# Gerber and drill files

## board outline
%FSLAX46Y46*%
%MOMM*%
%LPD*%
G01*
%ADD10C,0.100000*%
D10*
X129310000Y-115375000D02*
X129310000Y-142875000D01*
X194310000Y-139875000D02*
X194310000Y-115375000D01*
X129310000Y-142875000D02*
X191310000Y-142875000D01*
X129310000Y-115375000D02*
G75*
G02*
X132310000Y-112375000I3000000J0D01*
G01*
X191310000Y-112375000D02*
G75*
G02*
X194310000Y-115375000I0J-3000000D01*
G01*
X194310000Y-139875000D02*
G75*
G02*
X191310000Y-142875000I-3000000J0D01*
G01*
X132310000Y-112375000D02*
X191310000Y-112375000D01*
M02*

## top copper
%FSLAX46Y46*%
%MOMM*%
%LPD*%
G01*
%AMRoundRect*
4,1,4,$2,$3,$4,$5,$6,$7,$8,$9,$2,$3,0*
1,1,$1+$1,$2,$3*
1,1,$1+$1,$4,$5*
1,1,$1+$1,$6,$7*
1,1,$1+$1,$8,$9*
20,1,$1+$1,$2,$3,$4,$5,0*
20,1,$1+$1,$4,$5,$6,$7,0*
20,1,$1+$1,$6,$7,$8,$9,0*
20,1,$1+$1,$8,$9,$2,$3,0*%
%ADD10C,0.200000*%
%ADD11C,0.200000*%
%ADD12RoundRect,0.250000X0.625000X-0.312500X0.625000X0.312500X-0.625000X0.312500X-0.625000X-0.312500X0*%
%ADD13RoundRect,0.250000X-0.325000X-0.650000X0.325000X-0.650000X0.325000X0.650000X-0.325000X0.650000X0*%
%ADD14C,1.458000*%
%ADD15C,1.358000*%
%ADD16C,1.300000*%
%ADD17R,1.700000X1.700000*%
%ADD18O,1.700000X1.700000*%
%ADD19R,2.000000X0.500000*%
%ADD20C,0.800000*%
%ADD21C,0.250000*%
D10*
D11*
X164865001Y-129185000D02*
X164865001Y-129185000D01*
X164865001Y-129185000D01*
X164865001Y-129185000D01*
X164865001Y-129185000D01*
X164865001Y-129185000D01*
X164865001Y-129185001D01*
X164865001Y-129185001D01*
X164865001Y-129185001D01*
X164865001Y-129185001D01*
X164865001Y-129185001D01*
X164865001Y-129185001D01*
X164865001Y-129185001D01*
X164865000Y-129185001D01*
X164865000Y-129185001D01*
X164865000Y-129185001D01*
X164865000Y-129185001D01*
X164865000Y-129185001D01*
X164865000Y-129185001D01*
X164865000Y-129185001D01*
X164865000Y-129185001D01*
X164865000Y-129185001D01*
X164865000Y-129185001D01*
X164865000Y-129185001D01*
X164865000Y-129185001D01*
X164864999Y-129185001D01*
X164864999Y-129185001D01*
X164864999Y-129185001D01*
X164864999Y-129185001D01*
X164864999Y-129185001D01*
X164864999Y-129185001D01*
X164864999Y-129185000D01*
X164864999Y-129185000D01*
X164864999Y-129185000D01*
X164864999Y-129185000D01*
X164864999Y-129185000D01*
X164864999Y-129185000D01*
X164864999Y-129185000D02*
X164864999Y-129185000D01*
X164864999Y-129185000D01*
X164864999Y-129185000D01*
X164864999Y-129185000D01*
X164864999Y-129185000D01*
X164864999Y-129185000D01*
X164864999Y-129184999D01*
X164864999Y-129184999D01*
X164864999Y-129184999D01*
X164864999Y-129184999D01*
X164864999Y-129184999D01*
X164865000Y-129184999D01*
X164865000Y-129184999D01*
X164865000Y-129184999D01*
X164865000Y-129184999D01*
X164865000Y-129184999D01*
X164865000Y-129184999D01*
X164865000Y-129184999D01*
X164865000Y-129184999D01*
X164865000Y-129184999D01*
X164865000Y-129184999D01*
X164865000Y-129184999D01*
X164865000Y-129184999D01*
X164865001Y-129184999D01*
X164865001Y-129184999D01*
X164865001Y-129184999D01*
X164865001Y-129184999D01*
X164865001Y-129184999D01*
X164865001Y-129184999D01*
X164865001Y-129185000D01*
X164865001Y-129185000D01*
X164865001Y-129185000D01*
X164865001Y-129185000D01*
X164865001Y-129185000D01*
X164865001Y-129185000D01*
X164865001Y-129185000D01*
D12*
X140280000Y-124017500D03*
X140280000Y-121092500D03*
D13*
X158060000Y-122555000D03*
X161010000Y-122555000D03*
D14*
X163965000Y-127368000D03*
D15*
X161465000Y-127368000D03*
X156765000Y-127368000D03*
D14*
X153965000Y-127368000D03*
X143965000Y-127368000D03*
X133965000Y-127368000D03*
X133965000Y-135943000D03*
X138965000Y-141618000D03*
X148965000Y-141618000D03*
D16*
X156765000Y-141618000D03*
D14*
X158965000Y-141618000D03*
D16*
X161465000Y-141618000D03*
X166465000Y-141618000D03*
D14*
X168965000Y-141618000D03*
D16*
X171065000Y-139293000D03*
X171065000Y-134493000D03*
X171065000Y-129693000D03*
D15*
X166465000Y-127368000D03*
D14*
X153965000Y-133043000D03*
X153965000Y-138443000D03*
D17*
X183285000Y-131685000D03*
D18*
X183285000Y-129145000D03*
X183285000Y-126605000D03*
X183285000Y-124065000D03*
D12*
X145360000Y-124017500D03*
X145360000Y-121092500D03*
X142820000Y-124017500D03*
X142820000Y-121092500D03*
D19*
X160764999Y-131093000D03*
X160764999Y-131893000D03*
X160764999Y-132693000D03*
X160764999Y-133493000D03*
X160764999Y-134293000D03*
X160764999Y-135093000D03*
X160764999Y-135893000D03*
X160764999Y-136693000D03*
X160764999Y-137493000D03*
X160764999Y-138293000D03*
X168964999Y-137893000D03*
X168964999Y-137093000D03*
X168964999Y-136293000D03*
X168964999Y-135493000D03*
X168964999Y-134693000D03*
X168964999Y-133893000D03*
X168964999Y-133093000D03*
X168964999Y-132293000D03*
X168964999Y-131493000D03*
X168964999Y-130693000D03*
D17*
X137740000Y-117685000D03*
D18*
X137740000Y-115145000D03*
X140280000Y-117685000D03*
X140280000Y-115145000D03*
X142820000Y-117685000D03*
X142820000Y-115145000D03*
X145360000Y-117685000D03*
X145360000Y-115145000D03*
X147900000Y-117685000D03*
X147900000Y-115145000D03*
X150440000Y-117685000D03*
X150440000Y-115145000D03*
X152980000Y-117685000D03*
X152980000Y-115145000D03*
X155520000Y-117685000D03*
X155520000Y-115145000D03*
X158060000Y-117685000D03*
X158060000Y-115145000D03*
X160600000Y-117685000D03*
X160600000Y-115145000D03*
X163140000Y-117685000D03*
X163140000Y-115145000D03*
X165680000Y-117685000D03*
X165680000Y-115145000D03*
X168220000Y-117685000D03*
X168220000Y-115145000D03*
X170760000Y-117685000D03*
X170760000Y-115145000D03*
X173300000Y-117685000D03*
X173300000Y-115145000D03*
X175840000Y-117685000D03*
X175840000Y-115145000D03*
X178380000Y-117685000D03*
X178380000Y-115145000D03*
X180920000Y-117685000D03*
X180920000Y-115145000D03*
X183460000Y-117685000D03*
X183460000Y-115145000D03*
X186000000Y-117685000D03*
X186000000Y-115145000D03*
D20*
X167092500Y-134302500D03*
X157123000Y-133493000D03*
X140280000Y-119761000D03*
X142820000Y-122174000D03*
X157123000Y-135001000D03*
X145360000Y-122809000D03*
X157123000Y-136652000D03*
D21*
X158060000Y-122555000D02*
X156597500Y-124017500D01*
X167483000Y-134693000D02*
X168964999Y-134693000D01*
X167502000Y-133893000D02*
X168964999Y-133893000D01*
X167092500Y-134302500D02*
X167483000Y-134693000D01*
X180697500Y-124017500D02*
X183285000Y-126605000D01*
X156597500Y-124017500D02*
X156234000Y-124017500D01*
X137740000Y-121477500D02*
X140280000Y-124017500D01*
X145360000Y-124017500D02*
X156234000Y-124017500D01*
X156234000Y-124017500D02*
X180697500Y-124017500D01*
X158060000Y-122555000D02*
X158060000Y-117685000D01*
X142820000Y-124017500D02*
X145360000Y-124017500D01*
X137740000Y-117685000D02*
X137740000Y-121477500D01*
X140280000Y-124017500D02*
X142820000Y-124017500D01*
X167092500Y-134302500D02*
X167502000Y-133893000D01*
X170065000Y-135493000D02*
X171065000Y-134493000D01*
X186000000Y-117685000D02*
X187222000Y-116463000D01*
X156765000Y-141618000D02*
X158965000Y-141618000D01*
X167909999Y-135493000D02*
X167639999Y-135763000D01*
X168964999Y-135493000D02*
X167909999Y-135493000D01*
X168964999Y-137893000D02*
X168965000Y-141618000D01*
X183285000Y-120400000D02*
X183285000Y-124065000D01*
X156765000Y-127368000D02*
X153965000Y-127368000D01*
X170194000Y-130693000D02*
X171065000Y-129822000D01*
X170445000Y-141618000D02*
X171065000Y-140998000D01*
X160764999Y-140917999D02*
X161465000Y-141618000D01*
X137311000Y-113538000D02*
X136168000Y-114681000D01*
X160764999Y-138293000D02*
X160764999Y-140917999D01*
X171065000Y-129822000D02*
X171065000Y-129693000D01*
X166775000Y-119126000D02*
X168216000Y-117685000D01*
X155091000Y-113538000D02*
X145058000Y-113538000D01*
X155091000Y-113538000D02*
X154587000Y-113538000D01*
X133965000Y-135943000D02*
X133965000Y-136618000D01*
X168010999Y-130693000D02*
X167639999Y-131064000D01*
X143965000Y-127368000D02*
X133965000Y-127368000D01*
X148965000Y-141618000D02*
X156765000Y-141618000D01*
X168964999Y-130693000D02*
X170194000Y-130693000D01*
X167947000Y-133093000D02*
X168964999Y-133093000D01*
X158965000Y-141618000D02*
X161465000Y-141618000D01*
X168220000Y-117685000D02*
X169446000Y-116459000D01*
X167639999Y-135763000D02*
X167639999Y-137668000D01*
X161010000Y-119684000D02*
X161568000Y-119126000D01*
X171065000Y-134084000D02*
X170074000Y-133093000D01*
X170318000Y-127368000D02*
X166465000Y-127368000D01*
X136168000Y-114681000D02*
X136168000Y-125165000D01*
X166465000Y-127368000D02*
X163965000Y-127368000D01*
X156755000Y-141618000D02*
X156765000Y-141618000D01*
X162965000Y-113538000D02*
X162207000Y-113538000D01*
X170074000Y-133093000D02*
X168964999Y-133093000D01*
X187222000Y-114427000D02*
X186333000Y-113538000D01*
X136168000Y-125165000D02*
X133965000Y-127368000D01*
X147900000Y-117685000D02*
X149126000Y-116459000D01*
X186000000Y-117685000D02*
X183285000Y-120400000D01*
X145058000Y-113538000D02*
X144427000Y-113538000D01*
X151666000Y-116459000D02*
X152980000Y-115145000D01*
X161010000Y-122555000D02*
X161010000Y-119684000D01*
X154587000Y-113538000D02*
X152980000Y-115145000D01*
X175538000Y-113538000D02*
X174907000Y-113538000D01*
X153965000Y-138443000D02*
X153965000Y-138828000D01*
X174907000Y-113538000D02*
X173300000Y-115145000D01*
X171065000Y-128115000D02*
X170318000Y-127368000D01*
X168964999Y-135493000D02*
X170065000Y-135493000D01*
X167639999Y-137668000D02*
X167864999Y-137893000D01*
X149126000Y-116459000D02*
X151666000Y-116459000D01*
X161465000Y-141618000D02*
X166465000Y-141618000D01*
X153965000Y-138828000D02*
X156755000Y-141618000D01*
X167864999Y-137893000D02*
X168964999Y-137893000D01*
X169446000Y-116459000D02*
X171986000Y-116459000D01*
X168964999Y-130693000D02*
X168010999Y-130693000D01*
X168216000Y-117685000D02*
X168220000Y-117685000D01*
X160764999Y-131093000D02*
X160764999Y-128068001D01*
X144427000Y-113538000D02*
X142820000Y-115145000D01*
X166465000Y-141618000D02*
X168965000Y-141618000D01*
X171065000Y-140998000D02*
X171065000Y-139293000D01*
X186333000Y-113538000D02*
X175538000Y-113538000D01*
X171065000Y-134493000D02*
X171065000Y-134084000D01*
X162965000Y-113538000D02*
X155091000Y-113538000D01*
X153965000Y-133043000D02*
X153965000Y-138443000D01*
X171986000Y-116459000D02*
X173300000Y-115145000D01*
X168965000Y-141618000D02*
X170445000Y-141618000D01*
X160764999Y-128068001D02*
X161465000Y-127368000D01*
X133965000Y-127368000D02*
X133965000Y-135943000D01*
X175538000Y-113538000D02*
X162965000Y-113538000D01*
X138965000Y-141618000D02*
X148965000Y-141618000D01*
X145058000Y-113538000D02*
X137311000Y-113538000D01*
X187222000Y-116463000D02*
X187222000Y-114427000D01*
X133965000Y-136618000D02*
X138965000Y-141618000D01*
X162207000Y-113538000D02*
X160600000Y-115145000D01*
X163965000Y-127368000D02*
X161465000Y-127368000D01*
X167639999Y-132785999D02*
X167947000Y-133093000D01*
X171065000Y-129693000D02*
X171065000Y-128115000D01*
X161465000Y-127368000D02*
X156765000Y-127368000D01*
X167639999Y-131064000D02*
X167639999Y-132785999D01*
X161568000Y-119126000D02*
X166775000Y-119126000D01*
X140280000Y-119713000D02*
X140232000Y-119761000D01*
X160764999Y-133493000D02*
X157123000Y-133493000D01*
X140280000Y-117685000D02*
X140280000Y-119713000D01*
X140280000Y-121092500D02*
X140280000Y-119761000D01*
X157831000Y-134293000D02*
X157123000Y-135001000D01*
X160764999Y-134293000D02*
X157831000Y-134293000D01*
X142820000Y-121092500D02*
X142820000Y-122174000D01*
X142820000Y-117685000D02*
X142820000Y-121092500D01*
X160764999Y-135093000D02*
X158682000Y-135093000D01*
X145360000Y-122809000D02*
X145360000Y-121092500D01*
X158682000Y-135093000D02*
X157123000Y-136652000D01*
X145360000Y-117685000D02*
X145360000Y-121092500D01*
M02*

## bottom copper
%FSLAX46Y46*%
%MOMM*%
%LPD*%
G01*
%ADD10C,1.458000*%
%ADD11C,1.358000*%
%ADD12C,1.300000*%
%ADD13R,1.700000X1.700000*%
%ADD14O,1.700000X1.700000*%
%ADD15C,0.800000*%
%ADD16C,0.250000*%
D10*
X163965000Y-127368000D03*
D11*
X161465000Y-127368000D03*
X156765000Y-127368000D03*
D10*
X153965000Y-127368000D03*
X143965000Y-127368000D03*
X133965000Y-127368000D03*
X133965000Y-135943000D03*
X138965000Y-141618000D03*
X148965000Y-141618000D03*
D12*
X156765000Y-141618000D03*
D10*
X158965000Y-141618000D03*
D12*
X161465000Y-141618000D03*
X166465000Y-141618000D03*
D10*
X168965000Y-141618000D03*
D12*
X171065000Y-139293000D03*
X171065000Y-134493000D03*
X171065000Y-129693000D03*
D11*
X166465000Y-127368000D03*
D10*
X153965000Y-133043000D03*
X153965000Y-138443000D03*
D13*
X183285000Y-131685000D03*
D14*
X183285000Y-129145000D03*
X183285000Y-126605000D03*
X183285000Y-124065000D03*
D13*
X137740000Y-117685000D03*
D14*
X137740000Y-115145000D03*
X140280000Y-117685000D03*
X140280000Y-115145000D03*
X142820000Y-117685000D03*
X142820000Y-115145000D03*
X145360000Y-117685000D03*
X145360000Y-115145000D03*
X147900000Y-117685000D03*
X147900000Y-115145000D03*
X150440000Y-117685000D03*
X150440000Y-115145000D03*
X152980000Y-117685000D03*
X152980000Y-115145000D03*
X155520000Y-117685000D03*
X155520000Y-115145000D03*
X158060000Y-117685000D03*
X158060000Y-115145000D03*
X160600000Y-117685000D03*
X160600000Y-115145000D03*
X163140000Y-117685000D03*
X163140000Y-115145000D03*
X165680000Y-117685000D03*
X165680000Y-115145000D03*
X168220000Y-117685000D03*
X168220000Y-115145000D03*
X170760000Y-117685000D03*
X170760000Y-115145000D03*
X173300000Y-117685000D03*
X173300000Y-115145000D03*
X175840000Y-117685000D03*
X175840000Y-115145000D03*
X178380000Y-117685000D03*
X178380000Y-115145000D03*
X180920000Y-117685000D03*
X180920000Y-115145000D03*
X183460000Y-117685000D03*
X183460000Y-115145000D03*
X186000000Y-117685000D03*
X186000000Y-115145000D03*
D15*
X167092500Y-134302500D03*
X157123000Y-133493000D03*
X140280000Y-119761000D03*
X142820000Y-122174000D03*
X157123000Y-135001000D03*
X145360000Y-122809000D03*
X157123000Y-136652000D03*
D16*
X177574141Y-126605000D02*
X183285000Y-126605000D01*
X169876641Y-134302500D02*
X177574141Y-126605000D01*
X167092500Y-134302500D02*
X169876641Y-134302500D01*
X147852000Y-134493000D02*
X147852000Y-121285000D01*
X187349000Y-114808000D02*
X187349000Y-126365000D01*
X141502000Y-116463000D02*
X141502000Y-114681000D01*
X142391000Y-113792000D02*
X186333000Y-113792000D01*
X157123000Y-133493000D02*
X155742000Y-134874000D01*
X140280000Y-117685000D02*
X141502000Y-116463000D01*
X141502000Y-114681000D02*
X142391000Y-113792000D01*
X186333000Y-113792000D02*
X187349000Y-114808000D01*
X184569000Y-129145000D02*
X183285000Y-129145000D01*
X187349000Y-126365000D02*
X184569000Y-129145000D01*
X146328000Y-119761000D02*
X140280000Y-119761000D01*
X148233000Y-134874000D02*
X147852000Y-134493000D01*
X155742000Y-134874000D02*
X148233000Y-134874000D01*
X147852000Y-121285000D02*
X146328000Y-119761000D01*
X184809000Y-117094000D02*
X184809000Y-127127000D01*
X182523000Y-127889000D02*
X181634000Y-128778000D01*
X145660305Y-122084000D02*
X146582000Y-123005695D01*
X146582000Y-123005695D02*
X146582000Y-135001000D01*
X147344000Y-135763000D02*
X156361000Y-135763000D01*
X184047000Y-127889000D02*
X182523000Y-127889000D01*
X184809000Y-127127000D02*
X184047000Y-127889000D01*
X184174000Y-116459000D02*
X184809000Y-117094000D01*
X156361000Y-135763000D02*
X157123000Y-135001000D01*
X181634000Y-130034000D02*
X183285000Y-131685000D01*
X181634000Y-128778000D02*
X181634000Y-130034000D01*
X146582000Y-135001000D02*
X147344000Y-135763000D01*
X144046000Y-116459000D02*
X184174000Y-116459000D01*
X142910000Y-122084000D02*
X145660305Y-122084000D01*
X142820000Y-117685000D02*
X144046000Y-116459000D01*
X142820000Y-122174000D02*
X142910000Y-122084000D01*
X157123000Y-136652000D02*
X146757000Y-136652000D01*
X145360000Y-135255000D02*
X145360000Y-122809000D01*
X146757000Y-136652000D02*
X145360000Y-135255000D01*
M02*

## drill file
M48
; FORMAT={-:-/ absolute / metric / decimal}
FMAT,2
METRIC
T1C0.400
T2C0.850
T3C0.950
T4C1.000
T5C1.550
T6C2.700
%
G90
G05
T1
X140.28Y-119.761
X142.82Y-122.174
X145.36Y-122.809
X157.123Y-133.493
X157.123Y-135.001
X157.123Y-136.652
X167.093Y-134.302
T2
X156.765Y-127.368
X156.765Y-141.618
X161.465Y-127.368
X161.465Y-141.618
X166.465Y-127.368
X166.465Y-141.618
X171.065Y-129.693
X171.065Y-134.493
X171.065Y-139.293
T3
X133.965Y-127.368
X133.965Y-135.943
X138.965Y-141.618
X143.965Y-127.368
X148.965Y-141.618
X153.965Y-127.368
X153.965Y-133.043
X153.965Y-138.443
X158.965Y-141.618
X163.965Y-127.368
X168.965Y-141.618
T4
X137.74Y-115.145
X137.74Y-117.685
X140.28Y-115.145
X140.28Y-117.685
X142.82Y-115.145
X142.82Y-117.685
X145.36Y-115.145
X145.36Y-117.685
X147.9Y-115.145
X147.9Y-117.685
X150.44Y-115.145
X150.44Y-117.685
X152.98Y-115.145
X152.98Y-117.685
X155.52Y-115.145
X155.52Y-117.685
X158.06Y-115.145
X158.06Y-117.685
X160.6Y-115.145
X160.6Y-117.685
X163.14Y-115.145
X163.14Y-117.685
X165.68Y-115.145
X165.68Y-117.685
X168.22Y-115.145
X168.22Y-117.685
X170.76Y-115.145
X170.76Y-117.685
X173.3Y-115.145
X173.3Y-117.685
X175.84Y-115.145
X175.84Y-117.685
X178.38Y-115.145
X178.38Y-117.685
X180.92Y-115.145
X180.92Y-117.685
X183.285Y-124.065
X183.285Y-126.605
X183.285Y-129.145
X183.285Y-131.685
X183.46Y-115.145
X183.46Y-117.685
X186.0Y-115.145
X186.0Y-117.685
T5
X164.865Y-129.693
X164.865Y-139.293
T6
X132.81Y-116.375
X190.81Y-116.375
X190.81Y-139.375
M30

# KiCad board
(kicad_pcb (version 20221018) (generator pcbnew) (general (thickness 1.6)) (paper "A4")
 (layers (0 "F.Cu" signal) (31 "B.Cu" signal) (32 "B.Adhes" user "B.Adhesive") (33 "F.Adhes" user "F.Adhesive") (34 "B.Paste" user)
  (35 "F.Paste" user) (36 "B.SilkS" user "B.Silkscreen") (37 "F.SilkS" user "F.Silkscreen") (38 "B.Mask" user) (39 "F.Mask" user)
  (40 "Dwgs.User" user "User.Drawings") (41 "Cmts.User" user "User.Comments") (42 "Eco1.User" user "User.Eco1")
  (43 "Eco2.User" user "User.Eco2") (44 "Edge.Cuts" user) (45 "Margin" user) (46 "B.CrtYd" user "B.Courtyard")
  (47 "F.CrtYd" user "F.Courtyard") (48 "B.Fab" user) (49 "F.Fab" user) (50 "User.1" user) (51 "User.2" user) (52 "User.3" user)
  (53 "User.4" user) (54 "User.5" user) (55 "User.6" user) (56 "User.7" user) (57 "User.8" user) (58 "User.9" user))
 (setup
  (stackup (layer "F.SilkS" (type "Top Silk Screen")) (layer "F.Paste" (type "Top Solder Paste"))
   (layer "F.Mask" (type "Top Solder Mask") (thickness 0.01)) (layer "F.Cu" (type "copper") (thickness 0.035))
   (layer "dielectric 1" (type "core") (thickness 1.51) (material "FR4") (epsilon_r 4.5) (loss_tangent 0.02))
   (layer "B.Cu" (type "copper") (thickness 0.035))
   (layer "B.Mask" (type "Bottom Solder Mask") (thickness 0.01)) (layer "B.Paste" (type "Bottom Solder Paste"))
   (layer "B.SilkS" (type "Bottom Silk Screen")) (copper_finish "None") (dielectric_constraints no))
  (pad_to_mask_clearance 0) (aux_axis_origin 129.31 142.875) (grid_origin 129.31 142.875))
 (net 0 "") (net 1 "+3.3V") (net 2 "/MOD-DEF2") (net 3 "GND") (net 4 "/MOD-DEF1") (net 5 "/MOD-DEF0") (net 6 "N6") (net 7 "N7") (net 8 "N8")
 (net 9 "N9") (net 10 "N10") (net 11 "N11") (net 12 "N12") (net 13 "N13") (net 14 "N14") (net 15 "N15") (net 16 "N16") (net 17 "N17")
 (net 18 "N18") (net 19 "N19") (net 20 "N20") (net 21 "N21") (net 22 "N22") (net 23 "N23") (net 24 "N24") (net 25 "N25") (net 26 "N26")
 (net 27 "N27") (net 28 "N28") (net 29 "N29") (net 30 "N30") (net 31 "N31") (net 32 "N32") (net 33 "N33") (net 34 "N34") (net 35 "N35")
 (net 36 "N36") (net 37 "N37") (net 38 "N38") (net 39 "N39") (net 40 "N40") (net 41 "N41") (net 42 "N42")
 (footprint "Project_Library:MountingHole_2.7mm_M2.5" (layer "F.Cu") (at 190.81 139.375)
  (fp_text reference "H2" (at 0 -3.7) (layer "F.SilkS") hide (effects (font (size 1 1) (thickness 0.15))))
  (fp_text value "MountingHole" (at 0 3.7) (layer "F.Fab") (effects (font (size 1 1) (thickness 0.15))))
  (pad "" np_thru_hole circle (at 0 0) (size 2.7 2.7) (drill 2.7) (layers "*.Cu" "*.Mask")))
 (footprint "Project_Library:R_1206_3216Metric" (layer "F.Cu") (at 140.28 122.555 90)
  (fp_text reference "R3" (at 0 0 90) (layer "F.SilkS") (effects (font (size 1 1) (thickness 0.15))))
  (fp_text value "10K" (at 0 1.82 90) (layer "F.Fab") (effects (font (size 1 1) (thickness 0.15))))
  (pad "1" smd roundrect (at -1.4625 0 90) (size 1.125 1.75) (layers "F.Cu" "F.Paste" "F.Mask") (roundrect_rratio 0.2222222222)
   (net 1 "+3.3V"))
  (pad "2" smd roundrect (at 1.4625 0 90) (size 1.125 1.75) (layers "F.Cu" "F.Paste" "F.Mask") (roundrect_rratio 0.2222222222)
   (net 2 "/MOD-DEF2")))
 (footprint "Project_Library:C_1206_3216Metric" (layer "F.Cu") (at 159.535 122.555)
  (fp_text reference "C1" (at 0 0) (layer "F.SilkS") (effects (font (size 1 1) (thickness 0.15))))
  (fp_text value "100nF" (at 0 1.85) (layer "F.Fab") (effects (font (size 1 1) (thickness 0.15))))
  (pad "1" smd roundrect (at -1.475 0) (size 1.15 1.8) (layers "F.Cu" "F.Paste" "F.Mask") (roundrect_rratio 0.2173913043) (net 1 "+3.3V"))
  (pad "2" smd roundrect (at 1.475 0) (size 1.15 1.8) (layers "F.Cu" "F.Paste" "F.Mask") (roundrect_rratio 0.2173913043) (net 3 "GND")))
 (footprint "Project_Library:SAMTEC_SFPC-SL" (layer "F.Cu") (at 164.865 129.698)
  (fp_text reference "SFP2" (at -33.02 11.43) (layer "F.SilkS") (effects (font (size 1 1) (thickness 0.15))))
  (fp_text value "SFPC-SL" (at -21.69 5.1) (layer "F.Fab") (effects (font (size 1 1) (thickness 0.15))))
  (pad "S1" thru_hole circle (at -0.9 -2.33 180) (size 1.458 1.458) (drill 0.95) (layers "*.Cu" "*.Mask") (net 3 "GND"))
  (pad "S2" thru_hole circle (at -3.4 -2.33 180) (size 1.358 1.358) (drill 0.85) (layers "*.Cu" "*.Mask") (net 3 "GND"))
  (pad "S3" thru_hole circle (at -8.1 -2.33 180) (size 1.358 1.358) (drill 0.85) (layers "*.Cu" "*.Mask") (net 3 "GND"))
  (pad "S4" thru_hole circle (at -10.9 -2.33 180) (size 1.458 1.458) (drill 0.95) (layers "*.Cu" "*.Mask") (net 3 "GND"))
  (pad "S5" thru_hole circle (at -20.9 -2.33 180) (size 1.458 1.458) (drill 0.95) (layers "*.Cu" "*.Mask") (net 3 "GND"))
  (pad "S6" thru_hole circle (at -30.9 -2.33 180) (size 1.458 1.458) (drill 0.95) (layers "*.Cu" "*.Mask") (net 3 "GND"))
  (pad "S7" thru_hole circle (at -30.9 6.245 180) (size 1.458 1.458) (drill 0.95) (layers "*.Cu" "*.Mask") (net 3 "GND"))
  (pad "S8" thru_hole circle (at -25.9 11.92 180) (size 1.458 1.458) (drill 0.95) (layers "*.Cu" "*.Mask") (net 3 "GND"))
  (pad "S9" thru_hole circle (at -15.9 11.92 180) (size 1.458 1.458) (drill 0.95) (layers "*.Cu" "*.Mask") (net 3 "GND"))
  (pad "S10" thru_hole circle (at -8.1 11.92 180) (size 1.3 1.3) (drill 0.85) (layers "*.Cu" "*.Mask") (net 3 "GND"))
  (pad "S11" thru_hole circle (at -5.9 11.92 180) (size 1.458 1.458) (drill 0.95) (layers "*.Cu" "*.Mask") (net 3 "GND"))
  (pad "S12" thru_hole circle (at -3.4 11.92 180) (size 1.3 1.3) (drill 0.85) (layers "*.Cu" "*.Mask") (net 3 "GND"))
  (pad "S13" thru_hole circle (at 1.6 11.92 180) (size 1.3 1.3) (drill 0.85) (layers "*.Cu" "*.Mask") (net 3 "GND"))
  (pad "S14" thru_hole circle (at 4.1 11.92 180) (size 1.458 1.458) (drill 0.95) (layers "*.Cu" "*.Mask") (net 3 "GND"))
  (pad "S15" thru_hole circle (at 6.2 9.595 180) (size 1.3 1.3) (drill 0.85) (layers "*.Cu" "*.Mask") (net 3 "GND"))
  (pad "S16" thru_hole circle (at 6.2 4.795 180) (size 1.3 1.3) (drill 0.85) (layers "*.Cu" "*.Mask") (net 3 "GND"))
  (pad "S17" thru_hole circle (at 6.2 -0.005 180) (size 1.3 1.3) (drill 0.85) (layers "*.Cu" "*.Mask") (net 3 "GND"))
  (pad "S18" thru_hole circle (at 1.6 -2.33 180) (size 1.358 1.358) (drill 0.85) (layers "*.Cu" "*.Mask") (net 3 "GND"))
  (pad "S19" thru_hole circle (at -10.9 3.345 180) (size 1.458 1.458) (drill 0.95) (layers "*.Cu" "*.Mask") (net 3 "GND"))
  (pad "S20" thru_hole circle (at -10.9 8.745 180) (size 1.458 1.458) (drill 0.95) (layers "*.Cu" "*.Mask") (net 3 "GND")))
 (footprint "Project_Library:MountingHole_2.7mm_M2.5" (layer "F.Cu") (at 132.81 116.375)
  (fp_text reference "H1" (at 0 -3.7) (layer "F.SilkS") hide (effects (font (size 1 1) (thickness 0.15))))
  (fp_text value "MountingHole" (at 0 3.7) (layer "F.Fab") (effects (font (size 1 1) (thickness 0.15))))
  (pad "" np_thru_hole circle (at 0 0) (size 2.7 2.7) (drill 2.7) (layers "*.Cu" "*.Mask")))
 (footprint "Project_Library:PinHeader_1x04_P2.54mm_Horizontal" (layer "F.Cu") (at 183.285 124.065)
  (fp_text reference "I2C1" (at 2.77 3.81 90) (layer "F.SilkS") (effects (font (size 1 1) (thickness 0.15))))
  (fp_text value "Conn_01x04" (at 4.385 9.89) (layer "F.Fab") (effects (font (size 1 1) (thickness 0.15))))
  (pad "1" thru_hole rect (at 0 7.62) (size 1.7 1.7) (drill 1) (layers "*.Cu" "*.Mask") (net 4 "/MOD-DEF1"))
  (pad "2" thru_hole oval (at 0 5.08) (size 1.7 1.7) (drill 1) (layers "*.Cu" "*.Mask") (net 2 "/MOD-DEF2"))
  (pad "3" thru_hole oval (at 0 2.54) (size 1.7 1.7) (drill 1) (layers "*.Cu" "*.Mask") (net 1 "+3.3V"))
  (pad "4" thru_hole oval (at 0 0) (size 1.7 1.7) (drill 1) (layers "*.Cu" "*.Mask") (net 3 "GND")))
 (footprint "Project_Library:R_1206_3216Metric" (layer "F.Cu") (at 145.36 122.555 90)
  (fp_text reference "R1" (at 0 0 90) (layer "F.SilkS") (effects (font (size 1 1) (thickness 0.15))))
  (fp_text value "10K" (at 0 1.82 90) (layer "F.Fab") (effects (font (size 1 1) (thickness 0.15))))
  (pad "1" smd roundrect (at -1.4625 0 90) (size 1.125 1.75) (layers "F.Cu" "F.Paste" "F.Mask") (roundrect_rratio 0.2222222222)
   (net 1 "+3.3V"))
  (pad "2" smd roundrect (at 1.4625 0 90) (size 1.125 1.75) (layers "F.Cu" "F.Paste" "F.Mask") (roundrect_rratio 0.2222222222)
   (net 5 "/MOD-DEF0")))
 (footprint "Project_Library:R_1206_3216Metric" (layer "F.Cu") (at 142.82 122.555 90)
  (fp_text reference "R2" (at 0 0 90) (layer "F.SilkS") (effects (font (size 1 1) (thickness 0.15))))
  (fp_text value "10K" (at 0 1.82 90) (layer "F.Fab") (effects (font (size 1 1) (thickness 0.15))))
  (pad "1" smd roundrect (at -1.4625 0 90) (size 1.125 1.75) (layers "F.Cu" "F.Paste" "F.Mask") (roundrect_rratio 0.2222222222)
   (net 1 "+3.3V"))
  (pad "2" smd roundrect (at 1.4625 0 90) (size 1.125 1.75) (layers "F.Cu" "F.Paste" "F.Mask") (roundrect_rratio 0.2222222222)
   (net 4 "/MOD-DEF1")))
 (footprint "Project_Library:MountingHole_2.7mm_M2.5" (layer "F.Cu") (at 190.81 116.375)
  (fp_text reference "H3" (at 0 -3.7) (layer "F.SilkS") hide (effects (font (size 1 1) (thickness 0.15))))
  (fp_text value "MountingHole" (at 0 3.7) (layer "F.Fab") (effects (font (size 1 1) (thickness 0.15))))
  (pad "" np_thru_hole circle (at 0 0) (size 2.7 2.7) (drill 2.7) (layers "*.Cu" "*.Mask")))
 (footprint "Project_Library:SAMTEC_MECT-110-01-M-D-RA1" (layer "F.Cu") (at 164.864999 129.693)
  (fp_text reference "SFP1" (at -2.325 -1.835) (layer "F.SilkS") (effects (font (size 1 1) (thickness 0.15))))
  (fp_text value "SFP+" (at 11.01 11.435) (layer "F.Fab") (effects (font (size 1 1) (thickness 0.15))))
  (pad "" np_thru_hole circle (at 0 0 270) (size 1.55 1.55) (drill 1.55) (layers "*.Cu" "*.Mask"))
  (pad "" np_thru_hole circle (at 0 9.6 270) (size 1.55 1.55) (drill 1.55) (layers "*.Cu" "*.Mask"))
  (pad "01" smd rect (at -4.1 1.4 270) (size 0.5 2) (layers "F.Cu" "F.Paste" "F.Mask") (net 3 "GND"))
  (pad "02" smd rect (at -4.1 2.2 270) (size 0.5 2) (layers "F.Cu" "F.Paste" "F.Mask") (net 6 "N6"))
  (pad "03" smd rect (at -4.1 3 270) (size 0.5 2) (layers "F.Cu" "F.Paste" "F.Mask") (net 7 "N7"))
  (pad "04" smd rect (at -4.1 3.8 270) (size 0.5 2) (layers "F.Cu" "F.Paste" "F.Mask") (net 2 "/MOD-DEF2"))
  (pad "05" smd rect (at -4.1 4.6 270) (size 0.5 2) (layers "F.Cu" "F.Paste" "F.Mask") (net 4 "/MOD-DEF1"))
  (pad "06" smd rect (at -4.1 5.4 270) (size 0.5 2) (layers "F.Cu" "F.Paste" "F.Mask") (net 5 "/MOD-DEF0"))
  (pad "07" smd rect (at -4.1 6.2 270) (size 0.5 2) (layers "F.Cu" "F.Paste" "F.Mask") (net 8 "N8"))
  (pad "08" smd rect (at -4.1 7 270) (size 0.5 2) (layers "F.Cu" "F.Paste" "F.Mask") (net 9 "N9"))
  (pad "09" smd rect (at -4.1 7.8 270) (size 0.5 2) (layers "F.Cu" "F.Paste" "F.Mask") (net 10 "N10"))
  (pad "10" smd rect (at -4.1 8.6 270) (size 0.5 2) (layers "F.Cu" "F.Paste" "F.Mask") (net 3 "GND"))
  (pad "11" smd rect (at 4.1 8.2 270) (size 0.5 2) (layers "F.Cu" "F.Paste" "F.Mask") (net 3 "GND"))
  (pad "12" smd rect (at 4.1 7.4 270) (size 0.5 2) (layers "F.Cu" "F.Paste" "F.Mask") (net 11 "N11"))
  (pad "13" smd rect (at 4.1 6.6 270) (size 0.5 2) (layers "F.Cu" "F.Paste" "F.Mask") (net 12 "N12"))
  (pad "14" smd rect (at 4.1 5.8 270) (size 0.5 2) (layers "F.Cu" "F.Paste" "F.Mask") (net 3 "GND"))
  (pad "15" smd rect (at 4.1 5 270) (size 0.5 2) (layers "F.Cu" "F.Paste" "F.Mask") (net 1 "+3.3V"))
  (pad "16" smd rect (at 4.1 4.2 270) (size 0.5 2) (layers "F.Cu" "F.Paste" "F.Mask") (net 1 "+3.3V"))
  (pad "17" smd rect (at 4.1 3.4 270) (size 0.5 2) (layers "F.Cu" "F.Paste" "F.Mask") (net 3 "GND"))
  (pad "18" smd rect (at 4.1 2.6 270) (size 0.5 2) (layers "F.Cu" "F.Paste" "F.Mask") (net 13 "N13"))
  (pad "19" smd rect (at 4.1 1.8 270) (size 0.5 2) (layers "F.Cu" "F.Paste" "F.Mask") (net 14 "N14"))
  (pad "20" smd rect (at 4.1 1 270) (size 0.5 2) (layers "F.Cu" "F.Paste" "F.Mask") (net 3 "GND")))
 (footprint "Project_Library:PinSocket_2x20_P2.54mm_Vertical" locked (layer "B.Cu") (at 161.81 116.375 180)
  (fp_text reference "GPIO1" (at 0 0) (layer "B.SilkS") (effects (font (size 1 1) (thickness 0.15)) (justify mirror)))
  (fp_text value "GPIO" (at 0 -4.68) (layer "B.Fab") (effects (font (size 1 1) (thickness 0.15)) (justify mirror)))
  (pad "1" thru_hole rect locked (at 24.07 -1.31 270) (size 1.7 1.7) (drill 1) (layers "*.Cu" "*.Mask") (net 1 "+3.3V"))
  (pad "2" thru_hole oval locked (at 24.07 1.23 270) (size 1.7 1.7) (drill 1) (layers "*.Cu" "*.Mask") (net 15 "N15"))
  (pad "3" thru_hole oval locked (at 21.53 -1.31 270) (size 1.7 1.7) (drill 1) (layers "*.Cu" "*.Mask") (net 2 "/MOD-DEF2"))
  (pad "4" thru_hole oval locked (at 21.53 1.23 270) (size 1.7 1.7) (drill 1) (layers "*.Cu" "*.Mask") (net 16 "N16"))
  (pad "5" thru_hole oval locked (at 18.99 -1.31 270) (size 1.7 1.7) (drill 1) (layers "*.Cu" "*.Mask") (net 4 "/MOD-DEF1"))
  (pad "6" thru_hole oval locked (at 18.99 1.23 270) (size 1.7 1.7) (drill 1) (layers "*.Cu" "*.Mask") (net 3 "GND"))
  (pad "7" thru_hole oval locked (at 16.45 -1.31 270) (size 1.7 1.7) (drill 1) (layers "*.Cu" "*.Mask") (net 5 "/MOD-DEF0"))
  (pad "8" thru_hole oval locked (at 16.45 1.23 270) (size 1.7 1.7) (drill 1) (layers "*.Cu" "*.Mask") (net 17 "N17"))
  (pad "9" thru_hole oval locked (at 13.91 -1.31 270) (size 1.7 1.7) (drill 1) (layers "*.Cu" "*.Mask") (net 3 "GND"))
  (pad "10" thru_hole oval locked (at 13.91 1.23 270) (size 1.7 1.7) (drill 1) (layers "*.Cu" "*.Mask") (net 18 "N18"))
  (pad "11" thru_hole oval locked (at 11.37 -1.31 270) (size 1.7 1.7) (drill 1) (layers "*.Cu" "*.Mask") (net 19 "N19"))
  (pad "12" thru_hole oval locked (at 11.37 1.23 270) (size 1.7 1.7) (drill 1) (layers "*.Cu" "*.Mask") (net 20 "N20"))
  (pad "13" thru_hole oval locked (at 8.83 -1.31 270) (size 1.7 1.7) (drill 1) (layers "*.Cu" "*.Mask") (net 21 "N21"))
  (pad "14" thru_hole oval locked (at 8.83 1.23 270) (size 1.7 1.7) (drill 1) (layers "*.Cu" "*.Mask") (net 3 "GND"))
  (pad "15" thru_hole oval locked (at 6.29 -1.31 270) (size 1.7 1.7) (drill 1) (layers "*.Cu" "*.Mask") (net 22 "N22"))
  (pad "16" thru_hole oval locked (at 6.29 1.23 270) (size 1.7 1.7) (drill 1) (layers "*.Cu" "*.Mask") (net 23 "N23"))
  (pad "17" thru_hole oval locked (at 3.75 -1.31 270) (size 1.7 1.7) (drill 1) (layers "*.Cu" "*.Mask") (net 1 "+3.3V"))
  (pad "18" thru_hole oval locked (at 3.75 1.23 270) (size 1.7 1.7) (drill 1) (layers "*.Cu" "*.Mask") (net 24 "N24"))
  (pad "19" thru_hole oval locked (at 1.21 -1.31 270) (size 1.7 1.7) (drill 1) (layers "*.Cu" "*.Mask") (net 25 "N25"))
  (pad "20" thru_hole oval locked (at 1.21 1.23 270) (size 1.7 1.7) (drill 1) (layers "*.Cu" "*.Mask") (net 3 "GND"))
  (pad "21" thru_hole oval locked (at -1.33 -1.31 270) (size 1.7 1.7) (drill 1) (layers "*.Cu" "*.Mask") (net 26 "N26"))
  (pad "22" thru_hole oval locked (at -1.33 1.23 270) (size 1.7 1.7) (drill 1) (layers "*.Cu" "*.Mask") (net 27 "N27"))
  (pad "23" thru_hole oval locked (at -3.87 -1.31 270) (size 1.7 1.7) (drill 1) (layers "*.Cu" "*.Mask") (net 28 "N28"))
  (pad "24" thru_hole oval locked (at -3.87 1.23 270) (size 1.7 1.7) (drill 1) (layers "*.Cu" "*.Mask") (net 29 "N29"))
  (pad "25" thru_hole oval locked (at -6.41 -1.31 270) (size 1.7 1.7) (drill 1) (layers "*.Cu" "*.Mask") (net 3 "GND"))
  (pad "26" thru_hole oval locked (at -6.41 1.23 270) (size 1.7 1.7) (drill 1) (layers "*.Cu" "*.Mask") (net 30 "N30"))
  (pad "27" thru_hole oval locked (at -8.95 -1.31 270) (size 1.7 1.7) (drill 1) (layers "*.Cu" "*.Mask") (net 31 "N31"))
  (pad "28" thru_hole oval locked (at -8.95 1.23 270) (size 1.7 1.7) (drill 1) (layers "*.Cu" "*.Mask") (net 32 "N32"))
  (pad "29" thru_hole oval locked (at -11.49 -1.31 270) (size 1.7 1.7) (drill 1) (layers "*.Cu" "*.Mask") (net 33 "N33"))
  (pad "30" thru_hole oval locked (at -11.49 1.23 270) (size 1.7 1.7) (drill 1) (layers "*.Cu" "*.Mask") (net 3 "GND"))
  (pad "31" thru_hole oval locked (at -14.03 -1.31 270) (size 1.7 1.7) (drill 1) (layers "*.Cu" "*.Mask") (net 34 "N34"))
  (pad "32" thru_hole oval locked (at -14.03 1.23 270) (size 1.7 1.7) (drill 1) (layers "*.Cu" "*.Mask") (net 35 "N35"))
  (pad "33" thru_hole oval locked (at -16.57 -1.31 270) (size 1.7 1.7) (drill 1) (layers "*.Cu" "*.Mask") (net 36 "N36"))
  (pad "34" thru_hole oval locked (at -16.57 1.23 270) (size 1.7 1.7) (drill 1) (layers "*.Cu" "*.Mask") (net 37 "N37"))
  (pad "35" thru_hole oval locked (at -19.11 -1.31 270) (size 1.7 1.7) (drill 1) (layers "*.Cu" "*.Mask") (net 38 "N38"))
  (pad "36" thru_hole oval locked (at -19.11 1.23 270) (size 1.7 1.7) (drill 1) (layers "*.Cu" "*.Mask") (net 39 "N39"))
  (pad "37" thru_hole oval locked (at -21.65 -1.31 270) (size 1.7 1.7) (drill 1) (layers "*.Cu" "*.Mask") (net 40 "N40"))
  (pad "38" thru_hole oval locked (at -21.65 1.23 270) (size 1.7 1.7) (drill 1) (layers "*.Cu" "*.Mask") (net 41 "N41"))
  (pad "39" thru_hole oval locked (at -24.19 -1.31 270) (size 1.7 1.7) (drill 1) (layers "*.Cu" "*.Mask") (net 3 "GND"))
  (pad "40" thru_hole oval locked (at -24.19 1.23 270) (size 1.7 1.7) (drill 1) (layers "*.Cu" "*.Mask") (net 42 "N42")))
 (gr_circle locked (center 164.865 129.185) (end 164.865001 129.185) (stroke (width 0.2) (type default)) (fill none) (layer "F.Cu"))
 (gr_line (start 129.31 115.375) (end 129.31 142.875) (stroke (width 0.1) (type solid)) (layer "Edge.Cuts"))
 (gr_line (start 194.31 139.875) (end 194.31 115.375) (stroke (width 0.1) (type solid)) (layer "Edge.Cuts"))
 (gr_line (start 129.31 142.875) (end 191.31 142.875) (stroke (width 0.1) (type solid)) (layer "Edge.Cuts"))
 (gr_arc (start 129.31 115.375) (mid 130.18868 113.25368) (end 132.31 112.375) (stroke (width 0.1) (type solid)) (layer "Edge.Cuts"))
 (gr_arc (start 191.31 112.375) (mid 193.43132 113.25368) (end 194.31 115.375) (stroke (width 0.1) (type solid)) (layer "Edge.Cuts"))
 (gr_arc (start 194.31 139.875) (mid 193.43132 141.99632) (end 191.31 142.875) (stroke (width 0.1) (type solid)) (layer "Edge.Cuts"))
 (gr_line (start 132.31 112.375) (end 191.31 112.375) (stroke (width 0.1) (type solid)) (layer "Edge.Cuts"))
 (segment (start 158.06 122.555) (end 156.5975 124.0175) (width 0.25) (layer "F.Cu") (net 1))
 (segment (start 167.483 134.693) (end 168.964999 134.693) (width 0.25) (layer "F.Cu") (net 1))
 (segment (start 167.502 133.893) (end 168.964999 133.893) (width 0.25) (layer "F.Cu") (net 1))
 (segment (start 167.0925 134.3025) (end 167.483 134.693) (width 0.25) (layer "F.Cu") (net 1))
 (segment (start 180.6975 124.0175) (end 183.285 126.605) (width 0.25) (layer "F.Cu") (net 1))
 (segment (start 156.5975 124.0175) (end 156.234 124.0175) (width 0.25) (layer "F.Cu") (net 1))
 (segment (start 137.74 121.4775) (end 140.28 124.0175) (width 0.25) (layer "F.Cu") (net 1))
 (segment (start 145.36 124.0175) (end 156.234 124.0175) (width 0.25) (layer "F.Cu") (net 1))
 (segment (start 156.234 124.0175) (end 180.6975 124.0175) (width 0.25) (layer "F.Cu") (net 1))
 (segment (start 158.06 122.555) (end 158.06 117.685) (width 0.25) (layer "F.Cu") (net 1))
 (segment (start 142.82 124.0175) (end 145.36 124.0175) (width 0.25) (layer "F.Cu") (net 1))
 (segment (start 137.74 117.685) (end 137.74 121.4775) (width 0.25) (layer "F.Cu") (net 1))
 (segment (start 140.28 124.0175) (end 142.82 124.0175) (width 0.25) (layer "F.Cu") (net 1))
 (segment (start 167.0925 134.3025) (end 167.502 133.893) (width 0.25) (layer "F.Cu") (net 1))
 (via (at 167.0925 134.3025) (size 0.8) (drill 0.4) (layers "F.Cu" "B.Cu") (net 1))
 (segment (start 177.574141 126.605) (end 183.285 126.605) (width 0.25) (layer "B.Cu") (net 1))
 (segment (start 169.876641 134.3025) (end 177.574141 126.605) (width 0.25) (layer "B.Cu") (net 1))
 (segment (start 167.0925 134.3025) (end 169.876641 134.3025) (width 0.25) (layer "B.Cu") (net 1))
 (segment (start 170.065 135.493) (end 171.065 134.493) (width 0.25) (layer "F.Cu") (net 3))
 (segment (start 186 117.685) (end 187.222 116.463) (width 0.25) (layer "F.Cu") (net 3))
 (segment (start 156.765 141.618) (end 158.965 141.618) (width 0.25) (layer "F.Cu") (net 3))
 (segment (start 167.909999 135.493) (end 167.639999 135.763) (width 0.25) (layer "F.Cu") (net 3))
 (segment (start 168.964999 135.493) (end 167.909999 135.493) (width 0.25) (layer "F.Cu") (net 3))
 (segment (start 168.964999 137.893) (end 168.965 141.618) (width 0.25) (layer "F.Cu") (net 3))
 (segment (start 183.285 120.4) (end 183.285 124.065) (width 0.25) (layer "F.Cu") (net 3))
 (segment (start 156.765 127.368) (end 153.965 127.368) (width 0.25) (layer "F.Cu") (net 3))
 (segment (start 170.194 130.693) (end 171.065 129.822) (width 0.25) (layer "F.Cu") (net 3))
 (segment (start 170.445 141.618) (end 171.065 140.998) (width 0.25) (layer "F.Cu") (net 3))
 (segment (start 160.764999 140.917999) (end 161.465 141.618) (width 0.25) (layer "F.Cu") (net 3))
 (segment (start 137.311 113.538) (end 136.168 114.681) (width 0.25) (layer "F.Cu") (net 3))
 (segment (start 160.764999 138.293) (end 160.764999 140.917999) (width 0.25) (layer "F.Cu") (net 3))
 (segment (start 171.065 129.822) (end 171.065 129.693) (width 0.25) (layer "F.Cu") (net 3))
 (segment (start 166.775 119.126) (end 168.216 117.685) (width 0.25) (layer "F.Cu") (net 3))
 (segment (start 155.091 113.538) (end 145.058 113.538) (width 0.25) (layer "F.Cu") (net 3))
 (segment (start 155.091 113.538) (end 154.587 113.538) (width 0.25) (layer "F.Cu") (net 3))
 (segment (start 133.965 135.943) (end 133.965 136.618) (width 0.25) (layer "F.Cu") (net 3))
 (segment (start 168.010999 130.693) (end 167.639999 131.064) (width 0.25) (layer "F.Cu") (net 3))
 (segment (start 143.965 127.368) (end 133.965 127.368) (width 0.25) (layer "F.Cu") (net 3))
 (segment (start 148.965 141.618) (end 156.765 141.618) (width 0.25) (layer "F.Cu") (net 3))
 (segment (start 168.964999 130.693) (end 170.194 130.693) (width 0.25) (layer "F.Cu") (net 3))
 (segment (start 167.947 133.093) (end 168.964999 133.093) (width 0.25) (layer "F.Cu") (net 3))
 (segment (start 158.965 141.618) (end 161.465 141.618) (width 0.25) (layer "F.Cu") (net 3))
 (segment (start 168.22 117.685) (end 169.446 116.459) (width 0.25) (layer "F.Cu") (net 3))
 (segment (start 167.639999 135.763) (end 167.639999 137.668) (width 0.25) (layer "F.Cu") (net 3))
 (segment (start 161.01 119.684) (end 161.568 119.126) (width 0.25) (layer "F.Cu") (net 3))
 (segment (start 171.065 134.084) (end 170.074 133.093) (width 0.25) (layer "F.Cu") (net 3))
 (segment (start 170.318 127.368) (end 166.465 127.368) (width 0.25) (layer "F.Cu") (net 3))
 (segment (start 136.168 114.681) (end 136.168 125.165) (width 0.25) (layer "F.Cu") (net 3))
 (segment (start 166.465 127.368) (end 163.965 127.368) (width 0.25) (layer "F.Cu") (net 3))
 (segment (start 156.755 141.618) (end 156.765 141.618) (width 0.25) (layer "F.Cu") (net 3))
 (segment (start 162.965 113.538) (end 162.207 113.538) (width 0.25) (layer "F.Cu") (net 3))
 (segment (start 170.074 133.093) (end 168.964999 133.093) (width 0.25) (layer "F.Cu") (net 3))
 (segment (start 187.222 114.427) (end 186.333 113.538) (width 0.25) (layer "F.Cu") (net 3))
 (segment (start 136.168 125.165) (end 133.965 127.368) (width 0.25) (layer "F.Cu") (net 3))
 (segment (start 147.9 117.685) (end 149.126 116.459) (width 0.25) (layer "F.Cu") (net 3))
 (segment (start 186 117.685) (end 183.285 120.4) (width 0.25) (layer "F.Cu") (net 3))
 (segment (start 145.058 113.538) (end 144.427 113.538) (width 0.25) (layer "F.Cu") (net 3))
 (segment (start 151.666 116.459) (end 152.98 115.145) (width 0.25) (layer "F.Cu") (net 3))
 (segment (start 161.01 122.555) (end 161.01 119.684) (width 0.25) (layer "F.Cu") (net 3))
 (segment (start 154.587 113.538) (end 152.98 115.145) (width 0.25) (layer "F.Cu") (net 3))
 (segment (start 175.538 113.538) (end 174.907 113.538) (width 0.25) (layer "F.Cu") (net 3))
 (segment (start 153.965 138.443) (end 153.965 138.828) (width 0.25) (layer "F.Cu") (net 3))
 (segment (start 174.907 113.538) (end 173.3 115.145) (width 0.25) (layer "F.Cu") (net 3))
 (segment (start 171.065 128.115) (end 170.318 127.368) (width 0.25) (layer "F.Cu") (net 3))
 (segment (start 168.964999 135.493) (end 170.065 135.493) (width 0.25) (layer "F.Cu") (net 3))
 (segment (start 167.639999 137.668) (end 167.864999 137.893) (width 0.25) (layer "F.Cu") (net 3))
 (segment (start 149.126 116.459) (end 151.666 116.459) (width 0.25) (layer "F.Cu") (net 3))
 (segment (start 161.465 141.618) (end 166.465 141.618) (width 0.25) (layer "F.Cu") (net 3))
 (segment (start 153.965 138.828) (end 156.755 141.618) (width 0.25) (layer "F.Cu") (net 3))
 (segment (start 167.864999 137.893) (end 168.964999 137.893) (width 0.25) (layer "F.Cu") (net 3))
 (segment (start 169.446 116.459) (end 171.986 116.459) (width 0.25) (layer "F.Cu") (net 3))
 (segment (start 168.964999 130.693) (end 168.010999 130.693) (width 0.25) (layer "F.Cu") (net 3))
 (segment (start 168.216 117.685) (end 168.22 117.685) (width 0.25) (layer "F.Cu") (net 3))
 (segment (start 160.764999 131.093) (end 160.764999 128.068001) (width 0.25) (layer "F.Cu") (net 3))
 (segment (start 144.427 113.538) (end 142.82 115.145) (width 0.25) (layer "F.Cu") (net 3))
 (segment (start 166.465 141.618) (end 168.965 141.618) (width 0.25) (layer "F.Cu") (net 3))
 (segment (start 171.065 140.998) (end 171.065 139.293) (width 0.25) (layer "F.Cu") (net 3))
 (segment (start 186.333 113.538) (end 175.538 113.538) (width 0.25) (layer "F.Cu") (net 3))
 (segment (start 171.065 134.493) (end 171.065 134.084) (width 0.25) (layer "F.Cu") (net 3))
 (segment (start 162.965 113.538) (end 155.091 113.538) (width 0.25) (layer "F.Cu") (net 3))
 (segment (start 153.965 133.043) (end 153.965 138.443) (width 0.25) (layer "F.Cu") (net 3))
 (segment (start 171.986 116.459) (end 173.3 115.145) (width 0.25) (layer "F.Cu") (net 3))
 (segment (start 168.965 141.618) (end 170.445 141.618) (width 0.25) (layer "F.Cu") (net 3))
 (segment (start 160.764999 128.068001) (end 161.465 127.368) (width 0.25) (layer "F.Cu") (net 3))
 (segment (start 133.965 127.368) (end 133.965 135.943) (width 0.25) (layer "F.Cu") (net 3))
 (segment (start 175.538 113.538) (end 162.965 113.538) (width 0.25) (layer "F.Cu") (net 3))
 (segment (start 138.965 141.618) (end 148.965 141.618) (width 0.25) (layer "F.Cu") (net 3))
 (segment (start 145.058 113.538) (end 137.311 113.538) (width 0.25) (layer "F.Cu") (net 3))
 (segment (start 187.222 116.463) (end 187.222 114.427) (width 0.25) (layer "F.Cu") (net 3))
 (segment (start 133.965 136.618) (end 138.965 141.618) (width 0.25) (layer "F.Cu") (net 3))
 (segment (start 162.207 113.538) (end 160.6 115.145) (width 0.25) (layer "F.Cu") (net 3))
 (segment (start 163.965 127.368) (end 161.465 127.368) (width 0.25) (layer "F.Cu") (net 3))
 (segment (start 167.639999 132.785999) (end 167.947 133.093) (width 0.25) (layer "F.Cu") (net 3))
 (segment (start 171.065 129.693) (end 171.065 128.115) (width 0.25) (layer "F.Cu") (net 3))
 (segment (start 161.465 127.368) (end 156.765 127.368) (width 0.25) (layer "F.Cu") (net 3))
 (segment (start 167.639999 131.064) (end 167.639999 132.785999) (width 0.25) (layer "F.Cu") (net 3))
 (segment (start 161.568 119.126) (end 166.775 119.126) (width 0.25) (layer "F.Cu") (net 3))
 (segment (start 140.28 119.713) (end 140.232 119.761) (width 0.25) (layer "F.Cu") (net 2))
 (segment (start 160.764999 133.493) (end 157.123 133.493) (width 0.25) (layer "F.Cu") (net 2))
 (segment (start 140.28 117.685) (end 140.28 119.713) (width 0.25) (layer "F.Cu") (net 2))
 (segment (start 140.28 121.0925) (end 140.28 119.761) (width 0.25) (layer "F.Cu") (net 2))
 (via (at 157.123 133.493) (size 0.8) (drill 0.4) (layers "F.Cu" "B.Cu") (free) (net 2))
 (via (at 140.28 119.761) (size 0.8) (drill 0.4) (layers "F.Cu" "B.Cu") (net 2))
 (segment (start 147.852 134.493) (end 147.852 121.285) (width 0.25) (layer "B.Cu") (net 2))
 (segment (start 187.349 114.808) (end 187.349 126.365) (width 0.25) (layer "B.Cu") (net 2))
 (segment (start 141.502 116.463) (end 141.502 114.681) (width 0.25) (layer "B.Cu") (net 2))
 (segment (start 142.391 113.792) (end 186.333 113.792) (width 0.25) (layer "B.Cu") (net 2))
 (segment (start 157.123 133.493) (end 155.742 134.874) (width 0.25) (layer "B.Cu") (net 2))
 (segment (start 140.28 117.685) (end 141.502 116.463) (width 0.25) (layer "B.Cu") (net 2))
 (segment (start 141.502 114.681) (end 142.391 113.792) (width 0.25) (layer "B.Cu") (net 2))
 (segment (start 186.333 113.792) (end 187.349 114.808) (width 0.25) (layer "B.Cu") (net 2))
 (segment (start 184.569 129.145) (end 183.285 129.145) (width 0.25) (layer "B.Cu") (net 2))
 (segment (start 187.349 126.365) (end 184.569 129.145) (width 0.25) (layer "B.Cu") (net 2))
 (segment (start 146.328 119.761) (end 140.28 119.761) (width 0.25) (layer "B.Cu") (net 2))
 (segment (start 148.233 134.874) (end 147.852 134.493) (width 0.25) (layer "B.Cu") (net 2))
 (segment (start 155.742 134.874) (end 148.233 134.874) (width 0.25) (layer "B.Cu") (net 2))
 (segment (start 147.852 121.285) (end 146.328 119.761) (width 0.25) (layer "B.Cu") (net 2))
 (segment (start 157.831 134.293) (end 157.123 135.001) (width 0.25) (layer "F.Cu") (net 4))
 (segment (start 160.764999 134.293) (end 157.831 134.293) (width 0.25) (layer "F.Cu") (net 4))
 (segment (start 142.82 121.0925) (end 142.82 122.174) (width 0.25) (layer "F.Cu") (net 4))
 (segment (start 142.82 117.685) (end 142.82 121.0925) (width 0.25) (layer "F.Cu") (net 4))
 (via (at 142.82 122.174) (size 0.8) (drill 0.4) (layers "F.Cu" "B.Cu") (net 4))
 (via (at 157.123 135.001) (size 0.8) (drill 0.4) (layers "F.Cu" "B.Cu") (free) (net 4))
 (segment (start 184.809 117.094) (end 184.809 127.127) (width 0.25) (layer "B.Cu") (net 4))
 (segment (start 182.523 127.889) (end 181.634 128.778) (width 0.25) (layer "B.Cu") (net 4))
 (segment (start 145.660305 122.084) (end 146.582 123.005695) (width 0.25) (layer "B.Cu") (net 4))
 (segment (start 146.582 123.005695) (end 146.582 135.001) (width 0.25) (layer "B.Cu") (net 4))
 (segment (start 147.344 135.763) (end 156.361 135.763) (width 0.25) (layer "B.Cu") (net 4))
 (segment (start 184.047 127.889) (end 182.523 127.889) (width 0.25) (layer "B.Cu") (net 4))
 (segment (start 184.809 127.127) (end 184.047 127.889) (width 0.25) (layer "B.Cu") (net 4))
 (segment (start 184.174 116.459) (end 184.809 117.094) (width 0.25) (layer "B.Cu") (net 4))
 (segment (start 156.361 135.763) (end 157.123 135.001) (width 0.25) (layer "B.Cu") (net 4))
 (segment (start 181.634 130.034) (end 183.285 131.685) (width 0.25) (layer "B.Cu") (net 4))
 (segment (start 181.634 128.778) (end 181.634 130.034) (width 0.25) (layer "B.Cu") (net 4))
 (segment (start 146.582 135.001) (end 147.344 135.763) (width 0.25) (layer "B.Cu") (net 4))
 (segment (start 144.046 116.459) (end 184.174 116.459) (width 0.25) (layer "B.Cu") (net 4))
 (segment (start 142.91 122.084) (end 145.660305 122.084) (width 0.25) (layer "B.Cu") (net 4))
 (segment (start 142.82 117.685) (end 144.046 116.459) (width 0.25) (layer "B.Cu") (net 4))
 (segment (start 142.82 122.174) (end 142.91 122.084) (width 0.25) (layer "B.Cu") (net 4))
 (segment (start 160.764999 135.093) (end 158.682 135.093) (width 0.25) (layer "F.Cu") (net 5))
 (segment (start 145.36 122.809) (end 145.36 121.0925) (width 0.25) (layer "F.Cu") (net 5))
 (segment (start 158.682 135.093) (end 157.123 136.652) (width 0.25) (layer "F.Cu") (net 5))
 (segment (start 145.36 117.685) (end 145.36 121.0925) (width 0.25) (layer "F.Cu") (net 5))
 (via (at 145.36 122.809) (size 0.8) (drill 0.4) (layers "F.Cu" "B.Cu") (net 5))
 (via (at 157.123 136.652) (size 0.8) (drill 0.4) (layers "F.Cu" "B.Cu") (free) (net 5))
 (segment (start 157.123 136.652) (end 146.757 136.652) (width 0.25) (layer "B.Cu") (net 5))
 (segment (start 145.36 135.255) (end 145.36 122.809) (width 0.25) (layer "B.Cu") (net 5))
 (segment (start 146.757 136.652) (end 145.36 135.255) (width 0.25) (layer "B.Cu") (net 5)))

